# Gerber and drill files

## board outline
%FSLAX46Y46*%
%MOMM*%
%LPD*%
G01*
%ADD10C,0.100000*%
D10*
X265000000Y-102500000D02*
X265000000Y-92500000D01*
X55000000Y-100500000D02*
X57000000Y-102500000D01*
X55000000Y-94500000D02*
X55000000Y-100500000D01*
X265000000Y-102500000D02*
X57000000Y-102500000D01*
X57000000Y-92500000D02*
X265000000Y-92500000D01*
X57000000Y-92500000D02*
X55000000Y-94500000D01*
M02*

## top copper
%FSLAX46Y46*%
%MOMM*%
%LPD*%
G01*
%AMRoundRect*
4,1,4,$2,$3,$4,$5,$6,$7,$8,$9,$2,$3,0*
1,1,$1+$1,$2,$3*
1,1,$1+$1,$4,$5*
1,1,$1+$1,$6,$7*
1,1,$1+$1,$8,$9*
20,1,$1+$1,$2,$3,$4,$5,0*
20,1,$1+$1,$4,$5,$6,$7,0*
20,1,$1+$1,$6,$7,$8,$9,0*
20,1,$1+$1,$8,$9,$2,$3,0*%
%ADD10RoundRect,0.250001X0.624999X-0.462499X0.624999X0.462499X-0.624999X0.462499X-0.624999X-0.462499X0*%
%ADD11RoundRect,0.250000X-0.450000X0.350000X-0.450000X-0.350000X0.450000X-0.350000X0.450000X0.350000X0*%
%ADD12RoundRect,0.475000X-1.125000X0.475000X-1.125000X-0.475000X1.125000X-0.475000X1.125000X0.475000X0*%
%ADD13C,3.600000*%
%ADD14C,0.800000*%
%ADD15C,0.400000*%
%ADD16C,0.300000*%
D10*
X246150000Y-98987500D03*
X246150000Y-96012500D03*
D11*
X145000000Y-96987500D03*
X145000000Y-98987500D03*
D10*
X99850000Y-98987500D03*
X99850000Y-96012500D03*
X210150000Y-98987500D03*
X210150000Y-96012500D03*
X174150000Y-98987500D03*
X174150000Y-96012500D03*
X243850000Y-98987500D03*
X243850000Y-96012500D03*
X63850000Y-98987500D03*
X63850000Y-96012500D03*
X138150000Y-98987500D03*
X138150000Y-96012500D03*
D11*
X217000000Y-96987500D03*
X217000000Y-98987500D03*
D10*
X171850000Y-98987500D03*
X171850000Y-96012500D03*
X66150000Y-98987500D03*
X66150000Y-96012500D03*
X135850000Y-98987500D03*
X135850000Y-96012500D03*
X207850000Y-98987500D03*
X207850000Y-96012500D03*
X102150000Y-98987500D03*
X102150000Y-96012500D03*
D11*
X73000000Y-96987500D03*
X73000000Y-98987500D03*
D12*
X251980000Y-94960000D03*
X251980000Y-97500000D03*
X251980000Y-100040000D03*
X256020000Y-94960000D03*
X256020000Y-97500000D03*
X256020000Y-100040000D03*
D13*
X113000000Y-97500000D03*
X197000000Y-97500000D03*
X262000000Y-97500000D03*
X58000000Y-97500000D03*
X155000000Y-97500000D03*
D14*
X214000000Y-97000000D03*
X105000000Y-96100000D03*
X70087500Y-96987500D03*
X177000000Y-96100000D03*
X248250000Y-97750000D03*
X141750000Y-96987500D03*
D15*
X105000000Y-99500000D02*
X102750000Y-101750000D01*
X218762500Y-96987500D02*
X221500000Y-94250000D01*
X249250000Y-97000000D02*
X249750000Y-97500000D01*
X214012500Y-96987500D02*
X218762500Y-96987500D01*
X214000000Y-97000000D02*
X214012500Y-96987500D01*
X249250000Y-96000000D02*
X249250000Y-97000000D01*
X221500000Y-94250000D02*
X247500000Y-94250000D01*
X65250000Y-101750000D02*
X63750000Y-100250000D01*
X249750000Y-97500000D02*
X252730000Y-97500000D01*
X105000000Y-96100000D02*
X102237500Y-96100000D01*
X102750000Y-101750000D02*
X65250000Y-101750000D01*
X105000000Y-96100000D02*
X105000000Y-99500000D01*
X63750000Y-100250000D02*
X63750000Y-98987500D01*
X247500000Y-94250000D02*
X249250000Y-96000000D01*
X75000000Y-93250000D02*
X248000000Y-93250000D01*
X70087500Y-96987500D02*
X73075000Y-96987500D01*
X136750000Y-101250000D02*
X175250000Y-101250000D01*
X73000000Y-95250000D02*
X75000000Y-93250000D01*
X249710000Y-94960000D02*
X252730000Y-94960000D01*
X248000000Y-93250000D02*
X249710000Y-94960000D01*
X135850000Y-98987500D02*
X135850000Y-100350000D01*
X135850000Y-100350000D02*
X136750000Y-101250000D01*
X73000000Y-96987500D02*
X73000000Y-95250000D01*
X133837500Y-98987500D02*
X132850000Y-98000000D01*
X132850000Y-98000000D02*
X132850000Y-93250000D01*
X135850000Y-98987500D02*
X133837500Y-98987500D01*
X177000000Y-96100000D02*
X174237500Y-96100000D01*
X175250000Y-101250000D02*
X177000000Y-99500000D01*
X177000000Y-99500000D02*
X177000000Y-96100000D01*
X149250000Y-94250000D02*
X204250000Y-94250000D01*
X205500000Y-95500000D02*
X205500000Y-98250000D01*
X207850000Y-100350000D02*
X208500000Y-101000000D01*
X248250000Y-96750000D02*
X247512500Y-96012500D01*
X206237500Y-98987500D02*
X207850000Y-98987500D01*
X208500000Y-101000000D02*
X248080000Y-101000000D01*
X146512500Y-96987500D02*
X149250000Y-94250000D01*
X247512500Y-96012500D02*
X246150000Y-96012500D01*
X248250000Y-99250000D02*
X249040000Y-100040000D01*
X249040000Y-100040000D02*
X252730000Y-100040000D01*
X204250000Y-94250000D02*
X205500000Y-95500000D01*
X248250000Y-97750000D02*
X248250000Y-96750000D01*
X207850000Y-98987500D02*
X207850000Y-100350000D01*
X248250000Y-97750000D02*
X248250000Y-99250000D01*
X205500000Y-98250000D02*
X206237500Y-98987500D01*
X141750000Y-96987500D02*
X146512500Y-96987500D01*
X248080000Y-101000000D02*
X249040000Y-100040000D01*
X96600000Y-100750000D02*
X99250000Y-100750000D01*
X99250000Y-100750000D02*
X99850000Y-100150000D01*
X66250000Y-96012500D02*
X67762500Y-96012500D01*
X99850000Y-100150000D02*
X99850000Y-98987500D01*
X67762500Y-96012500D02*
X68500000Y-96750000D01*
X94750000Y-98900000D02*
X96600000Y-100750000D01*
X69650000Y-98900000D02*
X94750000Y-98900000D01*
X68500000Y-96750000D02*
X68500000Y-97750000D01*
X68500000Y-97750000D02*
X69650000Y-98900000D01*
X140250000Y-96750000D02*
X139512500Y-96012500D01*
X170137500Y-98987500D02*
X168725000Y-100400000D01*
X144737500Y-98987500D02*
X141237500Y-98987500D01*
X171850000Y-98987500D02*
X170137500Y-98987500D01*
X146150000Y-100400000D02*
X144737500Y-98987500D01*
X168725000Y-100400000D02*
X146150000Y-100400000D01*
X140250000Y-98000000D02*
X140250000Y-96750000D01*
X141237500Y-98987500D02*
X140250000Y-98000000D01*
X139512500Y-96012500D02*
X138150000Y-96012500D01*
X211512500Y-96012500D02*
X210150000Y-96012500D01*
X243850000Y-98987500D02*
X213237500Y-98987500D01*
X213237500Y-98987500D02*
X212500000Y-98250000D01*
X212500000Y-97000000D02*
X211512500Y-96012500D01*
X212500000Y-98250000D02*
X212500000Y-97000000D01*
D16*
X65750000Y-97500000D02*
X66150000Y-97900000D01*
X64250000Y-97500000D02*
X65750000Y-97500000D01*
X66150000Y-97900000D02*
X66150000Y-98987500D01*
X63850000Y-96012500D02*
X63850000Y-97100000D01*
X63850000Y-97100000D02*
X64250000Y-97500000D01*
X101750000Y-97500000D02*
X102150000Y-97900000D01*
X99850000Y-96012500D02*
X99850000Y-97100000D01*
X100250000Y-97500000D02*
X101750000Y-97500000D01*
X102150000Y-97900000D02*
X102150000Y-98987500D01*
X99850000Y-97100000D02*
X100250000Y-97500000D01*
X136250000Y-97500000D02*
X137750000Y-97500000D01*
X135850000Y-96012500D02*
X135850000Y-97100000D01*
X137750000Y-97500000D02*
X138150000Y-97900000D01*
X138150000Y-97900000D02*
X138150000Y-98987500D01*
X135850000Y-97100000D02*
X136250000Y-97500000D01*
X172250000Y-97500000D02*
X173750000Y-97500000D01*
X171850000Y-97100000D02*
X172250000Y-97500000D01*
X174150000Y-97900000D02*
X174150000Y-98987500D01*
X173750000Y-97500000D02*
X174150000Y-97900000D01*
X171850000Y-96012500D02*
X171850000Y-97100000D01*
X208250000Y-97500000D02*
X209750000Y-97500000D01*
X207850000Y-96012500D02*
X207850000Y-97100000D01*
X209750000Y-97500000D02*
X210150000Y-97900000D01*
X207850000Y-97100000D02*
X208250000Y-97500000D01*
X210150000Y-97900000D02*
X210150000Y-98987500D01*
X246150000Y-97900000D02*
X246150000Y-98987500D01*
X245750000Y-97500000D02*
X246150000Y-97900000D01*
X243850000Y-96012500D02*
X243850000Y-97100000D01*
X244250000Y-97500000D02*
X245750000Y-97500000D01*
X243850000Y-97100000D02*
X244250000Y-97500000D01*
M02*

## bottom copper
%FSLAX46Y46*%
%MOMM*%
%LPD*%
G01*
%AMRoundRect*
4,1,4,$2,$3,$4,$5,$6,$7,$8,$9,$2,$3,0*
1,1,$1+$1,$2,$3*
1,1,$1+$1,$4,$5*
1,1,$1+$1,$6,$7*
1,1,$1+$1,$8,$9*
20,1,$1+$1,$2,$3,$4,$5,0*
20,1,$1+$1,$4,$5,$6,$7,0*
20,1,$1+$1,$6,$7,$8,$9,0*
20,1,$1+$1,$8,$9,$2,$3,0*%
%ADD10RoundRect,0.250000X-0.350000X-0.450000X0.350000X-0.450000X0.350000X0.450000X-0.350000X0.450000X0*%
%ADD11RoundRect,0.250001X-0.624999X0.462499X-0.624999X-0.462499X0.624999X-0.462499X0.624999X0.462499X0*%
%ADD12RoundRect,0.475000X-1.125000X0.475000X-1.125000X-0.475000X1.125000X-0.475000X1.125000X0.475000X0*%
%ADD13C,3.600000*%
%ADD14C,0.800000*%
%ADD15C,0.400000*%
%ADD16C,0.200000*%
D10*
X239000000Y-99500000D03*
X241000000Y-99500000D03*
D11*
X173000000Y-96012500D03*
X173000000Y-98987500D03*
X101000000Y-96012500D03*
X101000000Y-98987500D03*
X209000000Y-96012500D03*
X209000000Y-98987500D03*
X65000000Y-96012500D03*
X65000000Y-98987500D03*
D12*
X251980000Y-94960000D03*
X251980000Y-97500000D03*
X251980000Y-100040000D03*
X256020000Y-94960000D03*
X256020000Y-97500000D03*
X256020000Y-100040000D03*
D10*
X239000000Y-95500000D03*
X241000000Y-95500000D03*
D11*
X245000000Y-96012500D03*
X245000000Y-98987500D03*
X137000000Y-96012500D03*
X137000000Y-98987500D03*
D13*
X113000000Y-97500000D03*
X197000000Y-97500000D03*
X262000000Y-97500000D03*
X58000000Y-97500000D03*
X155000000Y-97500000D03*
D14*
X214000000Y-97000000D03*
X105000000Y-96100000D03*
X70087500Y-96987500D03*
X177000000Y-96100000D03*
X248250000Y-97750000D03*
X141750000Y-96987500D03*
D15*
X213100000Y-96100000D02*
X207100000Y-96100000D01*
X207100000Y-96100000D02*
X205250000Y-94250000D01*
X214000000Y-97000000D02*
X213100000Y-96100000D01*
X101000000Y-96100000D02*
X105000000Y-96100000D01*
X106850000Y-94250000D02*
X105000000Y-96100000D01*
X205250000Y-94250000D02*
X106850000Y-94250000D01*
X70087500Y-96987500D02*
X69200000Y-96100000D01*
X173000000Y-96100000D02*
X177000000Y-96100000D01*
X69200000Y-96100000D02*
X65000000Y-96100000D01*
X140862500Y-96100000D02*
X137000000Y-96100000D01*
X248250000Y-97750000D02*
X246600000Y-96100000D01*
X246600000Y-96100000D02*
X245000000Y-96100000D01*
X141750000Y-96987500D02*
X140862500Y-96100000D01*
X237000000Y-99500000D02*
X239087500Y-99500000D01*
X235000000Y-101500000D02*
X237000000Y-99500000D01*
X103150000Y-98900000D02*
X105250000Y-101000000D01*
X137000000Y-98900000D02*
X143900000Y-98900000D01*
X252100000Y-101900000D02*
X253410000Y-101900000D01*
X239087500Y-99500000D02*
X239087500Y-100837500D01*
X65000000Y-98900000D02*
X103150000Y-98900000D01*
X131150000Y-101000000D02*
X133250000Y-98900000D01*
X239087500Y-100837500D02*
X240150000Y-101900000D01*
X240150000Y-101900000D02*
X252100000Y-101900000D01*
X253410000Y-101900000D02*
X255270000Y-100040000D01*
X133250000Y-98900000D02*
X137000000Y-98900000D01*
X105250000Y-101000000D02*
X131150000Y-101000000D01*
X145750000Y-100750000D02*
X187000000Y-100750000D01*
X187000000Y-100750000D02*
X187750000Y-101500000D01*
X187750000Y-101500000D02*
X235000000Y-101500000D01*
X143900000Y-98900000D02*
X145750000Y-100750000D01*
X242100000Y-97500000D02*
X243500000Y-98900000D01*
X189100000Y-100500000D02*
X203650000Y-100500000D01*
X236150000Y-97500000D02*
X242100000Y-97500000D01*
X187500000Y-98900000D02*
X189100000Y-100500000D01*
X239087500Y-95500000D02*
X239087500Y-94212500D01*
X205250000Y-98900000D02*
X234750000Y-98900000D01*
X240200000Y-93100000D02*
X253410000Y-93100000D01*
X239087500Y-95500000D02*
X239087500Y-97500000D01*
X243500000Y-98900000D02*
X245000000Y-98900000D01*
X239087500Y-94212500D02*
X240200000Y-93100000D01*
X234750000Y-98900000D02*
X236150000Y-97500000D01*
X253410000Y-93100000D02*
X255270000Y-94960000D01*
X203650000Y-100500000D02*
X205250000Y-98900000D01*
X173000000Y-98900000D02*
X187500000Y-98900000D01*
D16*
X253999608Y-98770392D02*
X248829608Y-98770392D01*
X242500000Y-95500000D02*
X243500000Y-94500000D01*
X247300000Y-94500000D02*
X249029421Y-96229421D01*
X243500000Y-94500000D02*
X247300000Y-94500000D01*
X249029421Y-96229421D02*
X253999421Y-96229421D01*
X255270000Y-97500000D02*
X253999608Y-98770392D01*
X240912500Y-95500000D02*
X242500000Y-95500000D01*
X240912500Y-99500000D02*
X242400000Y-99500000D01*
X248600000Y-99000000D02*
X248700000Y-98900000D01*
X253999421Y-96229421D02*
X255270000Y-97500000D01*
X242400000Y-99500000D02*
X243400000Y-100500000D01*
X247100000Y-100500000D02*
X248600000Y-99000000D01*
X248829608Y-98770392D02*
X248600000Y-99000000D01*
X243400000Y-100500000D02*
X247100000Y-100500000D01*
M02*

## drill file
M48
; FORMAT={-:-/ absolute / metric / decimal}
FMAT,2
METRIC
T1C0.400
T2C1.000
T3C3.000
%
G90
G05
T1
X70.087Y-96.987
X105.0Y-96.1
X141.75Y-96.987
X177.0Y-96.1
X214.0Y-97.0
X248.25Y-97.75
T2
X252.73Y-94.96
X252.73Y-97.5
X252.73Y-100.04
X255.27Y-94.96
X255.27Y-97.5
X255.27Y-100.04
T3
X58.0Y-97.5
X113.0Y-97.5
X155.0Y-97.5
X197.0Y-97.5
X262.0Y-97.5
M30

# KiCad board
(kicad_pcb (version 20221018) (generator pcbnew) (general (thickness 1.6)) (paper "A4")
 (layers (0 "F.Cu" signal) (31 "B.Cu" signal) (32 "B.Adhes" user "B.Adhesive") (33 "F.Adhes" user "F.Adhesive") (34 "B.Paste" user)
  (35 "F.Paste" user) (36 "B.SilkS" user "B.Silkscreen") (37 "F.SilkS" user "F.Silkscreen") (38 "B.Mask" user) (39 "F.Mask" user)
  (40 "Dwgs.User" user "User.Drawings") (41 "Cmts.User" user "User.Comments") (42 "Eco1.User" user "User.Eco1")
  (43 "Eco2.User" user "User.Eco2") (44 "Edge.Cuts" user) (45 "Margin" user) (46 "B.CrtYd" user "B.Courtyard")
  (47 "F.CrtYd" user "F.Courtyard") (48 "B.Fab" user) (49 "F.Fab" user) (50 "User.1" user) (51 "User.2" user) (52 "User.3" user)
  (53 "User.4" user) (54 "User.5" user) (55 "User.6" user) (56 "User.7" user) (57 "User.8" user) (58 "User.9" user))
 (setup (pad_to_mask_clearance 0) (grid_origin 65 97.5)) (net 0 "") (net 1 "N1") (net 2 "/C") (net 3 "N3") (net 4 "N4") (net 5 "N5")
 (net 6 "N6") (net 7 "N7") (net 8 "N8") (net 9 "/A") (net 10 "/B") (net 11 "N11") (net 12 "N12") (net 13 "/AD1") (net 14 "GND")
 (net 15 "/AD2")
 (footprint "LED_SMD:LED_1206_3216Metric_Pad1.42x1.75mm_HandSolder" (layer "F.Cu") (at 246.15 97.5 90)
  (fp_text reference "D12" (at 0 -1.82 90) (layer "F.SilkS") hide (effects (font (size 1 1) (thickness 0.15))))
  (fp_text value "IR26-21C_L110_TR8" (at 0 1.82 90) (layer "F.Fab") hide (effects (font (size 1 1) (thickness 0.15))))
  (pad "1" smd roundrect (at -1.4875 0 90) (size 1.425 1.75) (layers "F.Cu" "F.Paste" "F.Mask") (roundrect_rratio 0.175439) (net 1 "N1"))
  (pad "2" smd roundrect (at 1.4875 0 90) (size 1.425 1.75) (layers "F.Cu" "F.Paste" "F.Mask") (roundrect_rratio 0.175439) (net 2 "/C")))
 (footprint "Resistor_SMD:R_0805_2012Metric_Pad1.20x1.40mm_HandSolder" (layer "F.Cu") (at 145 97.9875 -90)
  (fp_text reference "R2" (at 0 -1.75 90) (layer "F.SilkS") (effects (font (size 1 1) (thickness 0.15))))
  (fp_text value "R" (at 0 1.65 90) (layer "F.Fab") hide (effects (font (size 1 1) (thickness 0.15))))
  (pad "1" smd roundrect (at -1 0 270) (size 1.2 1.4) (layers "F.Cu" "F.Paste" "F.Mask") (roundrect_rratio 0.208333) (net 2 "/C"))
  (pad "2" smd roundrect (at 1 0 270) (size 1.2 1.4) (layers "F.Cu" "F.Paste" "F.Mask") (roundrect_rratio 0.208333) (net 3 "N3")))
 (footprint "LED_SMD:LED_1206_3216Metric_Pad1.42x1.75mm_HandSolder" (layer "F.Cu") (at 99.85 97.5 90)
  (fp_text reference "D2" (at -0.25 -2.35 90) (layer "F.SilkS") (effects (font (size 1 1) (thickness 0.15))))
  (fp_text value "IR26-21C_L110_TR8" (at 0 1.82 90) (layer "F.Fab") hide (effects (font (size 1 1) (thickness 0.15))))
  (pad "1" smd roundrect (at -1.4875 0 90) (size 1.425 1.75) (layers "F.Cu" "F.Paste" "F.Mask") (roundrect_rratio 0.175439) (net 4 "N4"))
  (pad "2" smd roundrect (at 1.4875 0 90) (size 1.425 1.75) (layers "F.Cu" "F.Paste" "F.Mask") (roundrect_rratio 0.175439) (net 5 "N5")))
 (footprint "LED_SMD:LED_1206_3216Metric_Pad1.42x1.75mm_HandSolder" (layer "F.Cu") (at 210.15 97.5 90)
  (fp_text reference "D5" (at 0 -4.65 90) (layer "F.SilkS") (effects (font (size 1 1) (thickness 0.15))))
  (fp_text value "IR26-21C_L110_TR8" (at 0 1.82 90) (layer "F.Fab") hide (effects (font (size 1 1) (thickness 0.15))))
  (pad "1" smd roundrect (at -1.4875 0 90) (size 1.425 1.75) (layers "F.Cu" "F.Paste" "F.Mask") (roundrect_rratio 0.175439) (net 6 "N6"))
  (pad "2" smd roundrect (at 1.4875 0 90) (size 1.425 1.75) (layers "F.Cu" "F.Paste" "F.Mask") (roundrect_rratio 0.175439) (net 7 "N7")))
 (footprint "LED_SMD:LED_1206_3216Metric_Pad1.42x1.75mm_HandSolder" (layer "F.Cu") (at 174.15 97.5 90)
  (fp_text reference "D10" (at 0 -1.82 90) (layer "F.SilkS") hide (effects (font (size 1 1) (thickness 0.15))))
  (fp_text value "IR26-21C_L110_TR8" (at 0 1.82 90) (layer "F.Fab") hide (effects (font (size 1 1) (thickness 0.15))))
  (pad "1" smd roundrect (at -1.4875 0 90) (size 1.425 1.75) (layers "F.Cu" "F.Paste" "F.Mask") (roundrect_rratio 0.175439) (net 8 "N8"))
  (pad "2" smd roundrect (at 1.4875 0 90) (size 1.425 1.75) (layers "F.Cu" "F.Paste" "F.Mask") (roundrect_rratio 0.175439) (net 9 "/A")))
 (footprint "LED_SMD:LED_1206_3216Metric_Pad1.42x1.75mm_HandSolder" (layer "F.Cu") (at 243.85 97.5 90)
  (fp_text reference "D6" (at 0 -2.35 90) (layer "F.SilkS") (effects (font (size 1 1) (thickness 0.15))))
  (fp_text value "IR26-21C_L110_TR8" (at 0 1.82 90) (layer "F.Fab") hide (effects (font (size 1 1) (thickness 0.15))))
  (pad "1" smd roundrect (at -1.4875 0 90) (size 1.425 1.75) (layers "F.Cu" "F.Paste" "F.Mask") (roundrect_rratio 0.175439) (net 7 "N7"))
  (pad "2" smd roundrect (at 1.4875 0 90) (size 1.425 1.75) (layers "F.Cu" "F.Paste" "F.Mask") (roundrect_rratio 0.175439) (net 1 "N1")))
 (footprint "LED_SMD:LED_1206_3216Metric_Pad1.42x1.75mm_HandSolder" (layer "F.Cu") (at 63.85 97.5 90)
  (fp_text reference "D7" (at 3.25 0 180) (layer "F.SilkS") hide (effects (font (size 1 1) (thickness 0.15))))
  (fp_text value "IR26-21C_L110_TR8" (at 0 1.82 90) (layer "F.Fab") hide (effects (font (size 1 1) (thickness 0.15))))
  (pad "1" smd roundrect (at -1.4875 0 90) (size 1.425 1.75) (layers "F.Cu" "F.Paste" "F.Mask") (roundrect_rratio 0.175439) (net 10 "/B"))
  (pad "2" smd roundrect (at 1.4875 0 90) (size 1.425 1.75) (layers "F.Cu" "F.Paste" "F.Mask") (roundrect_rratio 0.175439) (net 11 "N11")))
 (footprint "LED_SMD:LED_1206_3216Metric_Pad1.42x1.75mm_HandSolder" (layer "F.Cu") (at 138.15 97.5 90)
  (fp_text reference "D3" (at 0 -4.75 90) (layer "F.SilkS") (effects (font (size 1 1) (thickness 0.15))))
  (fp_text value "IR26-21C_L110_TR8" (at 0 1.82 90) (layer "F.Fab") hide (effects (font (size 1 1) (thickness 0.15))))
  (pad "1" smd roundrect (at -1.4875 0 90) (size 1.425 1.75) (layers "F.Cu" "F.Paste" "F.Mask") (roundrect_rratio 0.175439) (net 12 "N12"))
  (pad "2" smd roundrect (at 1.4875 0 90) (size 1.425 1.75) (layers "F.Cu" "F.Paste" "F.Mask") (roundrect_rratio 0.175439) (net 3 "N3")))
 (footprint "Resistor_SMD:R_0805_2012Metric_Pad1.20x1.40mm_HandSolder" (layer "F.Cu") (at 217 97.9875 -90)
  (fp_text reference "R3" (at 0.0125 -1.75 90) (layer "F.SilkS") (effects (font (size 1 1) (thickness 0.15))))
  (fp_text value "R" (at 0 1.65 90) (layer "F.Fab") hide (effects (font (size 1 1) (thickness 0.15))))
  (pad "1" smd roundrect (at -1 0 270) (size 1.2 1.4) (layers "F.Cu" "F.Paste" "F.Mask") (roundrect_rratio 0.208333) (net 10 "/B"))
  (pad "2" smd roundrect (at 1 0 270) (size 1.2 1.4) (layers "F.Cu" "F.Paste" "F.Mask") (roundrect_rratio 0.208333) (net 7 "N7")))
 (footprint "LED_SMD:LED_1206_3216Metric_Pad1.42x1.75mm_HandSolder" (layer "F.Cu") (at 171.85 97.5 90)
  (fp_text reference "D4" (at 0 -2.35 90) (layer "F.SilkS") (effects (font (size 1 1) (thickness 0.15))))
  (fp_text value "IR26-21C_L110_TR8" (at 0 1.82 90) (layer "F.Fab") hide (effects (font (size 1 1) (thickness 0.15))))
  (pad "1" smd roundrect (at -1.4875 0 90) (size 1.425 1.75) (layers "F.Cu" "F.Paste" "F.Mask") (roundrect_rratio 0.175439) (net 3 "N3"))
  (pad "2" smd roundrect (at 1.4875 0 90) (size 1.425 1.75) (layers "F.Cu" "F.Paste" "F.Mask") (roundrect_rratio 0.175439) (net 8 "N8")))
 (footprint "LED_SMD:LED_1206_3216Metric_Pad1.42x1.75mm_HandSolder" (layer "F.Cu") (at 66.15 97.5 90)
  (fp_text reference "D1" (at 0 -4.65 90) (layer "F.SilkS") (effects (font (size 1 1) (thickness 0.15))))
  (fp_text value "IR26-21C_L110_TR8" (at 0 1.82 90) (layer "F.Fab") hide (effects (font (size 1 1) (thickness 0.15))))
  (pad "1" smd roundrect (at -1.4875 0 90) (size 1.425 1.75) (layers "F.Cu" "F.Paste" "F.Mask") (roundrect_rratio 0.175439) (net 11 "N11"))
  (pad "2" smd roundrect (at 1.4875 0 90) (size 1.425 1.75) (layers "F.Cu" "F.Paste" "F.Mask") (roundrect_rratio 0.175439) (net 4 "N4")))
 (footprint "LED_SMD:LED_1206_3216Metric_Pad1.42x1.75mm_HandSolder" (layer "F.Cu") (at 135.85 97.5 90)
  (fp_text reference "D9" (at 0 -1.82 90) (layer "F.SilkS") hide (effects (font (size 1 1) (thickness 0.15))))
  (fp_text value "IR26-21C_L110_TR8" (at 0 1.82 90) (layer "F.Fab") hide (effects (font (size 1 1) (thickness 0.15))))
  (pad "1" smd roundrect (at -1.4875 0 90) (size 1.425 1.75) (layers "F.Cu" "F.Paste" "F.Mask") (roundrect_rratio 0.175439) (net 9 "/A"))
  (pad "2" smd roundrect (at 1.4875 0 90) (size 1.425 1.75) (layers "F.Cu" "F.Paste" "F.Mask") (roundrect_rratio 0.175439) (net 12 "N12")))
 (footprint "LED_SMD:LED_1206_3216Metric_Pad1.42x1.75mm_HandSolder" (layer "F.Cu") (at 207.85 97.5 90)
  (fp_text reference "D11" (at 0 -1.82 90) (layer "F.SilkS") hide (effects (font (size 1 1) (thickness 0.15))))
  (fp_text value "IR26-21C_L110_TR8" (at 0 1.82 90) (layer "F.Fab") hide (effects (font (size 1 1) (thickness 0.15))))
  (pad "1" smd roundrect (at -1.4875 0 90) (size 1.425 1.75) (layers "F.Cu" "F.Paste" "F.Mask") (roundrect_rratio 0.175439) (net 2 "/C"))
  (pad "2" smd roundrect (at 1.4875 0 90) (size 1.425 1.75) (layers "F.Cu" "F.Paste" "F.Mask") (roundrect_rratio 0.175439) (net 6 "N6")))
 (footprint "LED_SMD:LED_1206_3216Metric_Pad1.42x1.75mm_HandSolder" (layer "F.Cu") (at 102.15 97.5 90)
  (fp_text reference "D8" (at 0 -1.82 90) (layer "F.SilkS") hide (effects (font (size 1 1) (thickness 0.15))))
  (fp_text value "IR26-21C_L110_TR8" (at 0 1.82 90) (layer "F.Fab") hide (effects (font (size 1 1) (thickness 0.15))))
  (pad "1" smd roundrect (at -1.4875 0 90) (size 1.425 1.75) (layers "F.Cu" "F.Paste" "F.Mask") (roundrect_rratio 0.175439) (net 5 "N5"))
  (pad "2" smd roundrect (at 1.4875 0 90) (size 1.425 1.75) (layers "F.Cu" "F.Paste" "F.Mask") (roundrect_rratio 0.175439) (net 10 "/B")))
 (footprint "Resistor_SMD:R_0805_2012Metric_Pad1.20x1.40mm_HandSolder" (layer "F.Cu") (at 73 97.9875 -90)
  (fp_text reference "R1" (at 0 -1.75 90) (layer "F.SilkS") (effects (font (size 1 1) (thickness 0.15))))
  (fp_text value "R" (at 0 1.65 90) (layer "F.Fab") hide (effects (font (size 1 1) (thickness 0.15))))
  (pad "1" smd roundrect (at -1 0 270) (size 1.2 1.4) (layers "F.Cu" "F.Paste" "F.Mask") (roundrect_rratio 0.208333) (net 9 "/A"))
  (pad "2" smd roundrect (at 1 0 270) (size 1.2 1.4) (layers "F.Cu" "F.Paste" "F.Mask") (roundrect_rratio 0.208333) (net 4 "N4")))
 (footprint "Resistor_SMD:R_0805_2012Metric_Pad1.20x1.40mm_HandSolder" (layer "B.Cu") (at 240 99.5)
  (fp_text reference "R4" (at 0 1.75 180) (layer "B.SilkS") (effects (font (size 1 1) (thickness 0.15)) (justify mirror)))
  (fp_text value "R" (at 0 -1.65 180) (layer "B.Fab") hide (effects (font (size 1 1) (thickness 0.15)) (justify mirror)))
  (pad "1" smd roundrect (at -1 0) (size 1.2 1.4) (layers "B.Cu" "B.Paste" "B.Mask") (roundrect_rratio 0.208333) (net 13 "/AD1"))
  (pad "2" smd roundrect (at 1 0) (size 1.2 1.4) (layers "B.Cu" "B.Paste" "B.Mask") (roundrect_rratio 0.208333) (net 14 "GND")))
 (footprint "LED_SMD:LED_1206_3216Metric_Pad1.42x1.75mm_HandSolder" (layer "B.Cu") (at 173 97.5 -90)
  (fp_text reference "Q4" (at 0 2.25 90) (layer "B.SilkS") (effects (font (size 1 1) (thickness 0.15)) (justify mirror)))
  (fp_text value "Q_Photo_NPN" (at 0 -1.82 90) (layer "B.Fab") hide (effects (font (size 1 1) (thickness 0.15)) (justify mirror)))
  (pad "1" smd roundrect (at -1.4875 0 270) (size 1.425 1.75) (layers "B.Cu" "B.Paste" "B.Mask") (roundrect_rratio 0.175439) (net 9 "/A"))
  (pad "2" smd roundrect (at 1.4875 0 270) (size 1.425 1.75) (layers "B.Cu" "B.Paste" "B.Mask") (roundrect_rratio 0.175439) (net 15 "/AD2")))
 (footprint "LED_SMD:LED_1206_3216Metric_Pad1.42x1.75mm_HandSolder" (layer "B.Cu") (at 101 97.5 -90)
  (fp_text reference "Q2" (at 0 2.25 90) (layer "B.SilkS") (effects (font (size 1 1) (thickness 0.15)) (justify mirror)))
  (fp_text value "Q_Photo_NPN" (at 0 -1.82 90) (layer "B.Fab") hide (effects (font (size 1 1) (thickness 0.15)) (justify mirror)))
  (pad "1" smd roundrect (at -1.4875 0 270) (size 1.425 1.75) (layers "B.Cu" "B.Paste" "B.Mask") (roundrect_rratio 0.175439) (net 10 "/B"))
  (pad "2" smd roundrect (at 1.4875 0 270) (size 1.425 1.75) (layers "B.Cu" "B.Paste" "B.Mask") (roundrect_rratio 0.175439) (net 13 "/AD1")))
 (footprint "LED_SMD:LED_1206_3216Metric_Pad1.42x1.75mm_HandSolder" (layer "B.Cu") (at 209 97.5 -90)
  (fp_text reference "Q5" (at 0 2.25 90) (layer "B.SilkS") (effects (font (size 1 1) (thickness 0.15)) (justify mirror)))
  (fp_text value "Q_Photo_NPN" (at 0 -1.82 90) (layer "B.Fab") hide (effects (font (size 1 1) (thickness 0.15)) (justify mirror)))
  (pad "1" smd roundrect (at -1.4875 0 270) (size 1.425 1.75) (layers "B.Cu" "B.Paste" "B.Mask") (roundrect_rratio 0.175439) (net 10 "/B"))
  (pad "2" smd roundrect (at 1.4875 0 270) (size 1.425 1.75) (layers "B.Cu" "B.Paste" "B.Mask") (roundrect_rratio 0.175439) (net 15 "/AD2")))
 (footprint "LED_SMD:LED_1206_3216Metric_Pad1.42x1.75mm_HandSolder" (layer "B.Cu") (at 65 97.5 -90)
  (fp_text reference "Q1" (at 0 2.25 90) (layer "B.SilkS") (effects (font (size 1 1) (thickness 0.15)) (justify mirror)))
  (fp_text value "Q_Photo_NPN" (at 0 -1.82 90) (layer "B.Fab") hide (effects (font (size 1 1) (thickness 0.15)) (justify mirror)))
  (pad "1" smd roundrect (at -1.4875 0 270) (size 1.425 1.75) (layers "B.Cu" "B.Paste" "B.Mask") (roundrect_rratio 0.175439) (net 9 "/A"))
  (pad "2" smd roundrect (at 1.4875 0 270) (size 1.425 1.75) (layers "B.Cu" "B.Paste" "B.Mask") (roundrect_rratio 0.175439) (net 13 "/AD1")))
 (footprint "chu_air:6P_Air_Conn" (layer "B.Cu") (at 254 97.5 -90)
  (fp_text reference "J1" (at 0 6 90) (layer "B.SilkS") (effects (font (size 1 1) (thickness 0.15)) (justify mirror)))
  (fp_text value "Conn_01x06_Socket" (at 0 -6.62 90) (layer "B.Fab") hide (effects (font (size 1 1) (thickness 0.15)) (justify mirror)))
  (pad "1" thru_hole roundrect (at -2.54 1.27 270) (size 1.9 3.2) (drill 1 (offset 0 0.75)) (layers "*.Cu" "*.Mask") (roundrect_rratio 0.25)
   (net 9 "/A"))
  (pad "2" thru_hole roundrect (at 0 1.27 270) (size 1.9 3.2) (drill 1 (offset 0 0.75)) (layers "*.Cu" "*.Mask") (roundrect_rratio 0.25)
   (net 10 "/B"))
  (pad "3" thru_hole roundrect (at 2.54 1.27 270) (size 1.9 3.2) (drill 1 (offset 0 0.75)) (layers "*.Cu" "*.Mask") (roundrect_rratio 0.25)
   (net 2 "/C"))
  (pad "4" thru_hole roundrect (at -2.54 -1.27 270) (size 1.9 3.2) (drill 1 (offset 0 -0.75)) (layers "*.Cu" "*.Mask")
   (roundrect_rratio 0.25) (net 15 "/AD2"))
  (pad "5" thru_hole roundrect (at 0 -1.27 270) (size 1.9 3.2) (drill 1 (offset 0 -0.75)) (layers "*.Cu" "*.Mask") (roundrect_rratio 0.25)
   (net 14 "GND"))
  (pad "6" thru_hole roundrect (at 2.54 -1.27 270) (size 1.9 3.2) (drill 1 (offset 0 -0.75)) (layers "*.Cu" "*.Mask")
   (roundrect_rratio 0.25) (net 13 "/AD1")))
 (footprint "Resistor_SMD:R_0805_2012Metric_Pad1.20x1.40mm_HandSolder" (layer "B.Cu") (at 240 95.5)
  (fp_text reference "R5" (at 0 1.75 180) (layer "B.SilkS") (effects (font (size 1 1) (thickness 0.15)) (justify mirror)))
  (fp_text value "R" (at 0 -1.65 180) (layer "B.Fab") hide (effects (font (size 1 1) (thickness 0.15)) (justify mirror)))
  (pad "1" smd roundrect (at -1 0) (size 1.2 1.4) (layers "B.Cu" "B.Paste" "B.Mask") (roundrect_rratio 0.208333) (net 15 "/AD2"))
  (pad "2" smd roundrect (at 1 0) (size 1.2 1.4) (layers "B.Cu" "B.Paste" "B.Mask") (roundrect_rratio 0.208333) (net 14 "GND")))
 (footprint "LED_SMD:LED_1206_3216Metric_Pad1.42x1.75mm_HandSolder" (layer "B.Cu") (at 245 97.5 -90)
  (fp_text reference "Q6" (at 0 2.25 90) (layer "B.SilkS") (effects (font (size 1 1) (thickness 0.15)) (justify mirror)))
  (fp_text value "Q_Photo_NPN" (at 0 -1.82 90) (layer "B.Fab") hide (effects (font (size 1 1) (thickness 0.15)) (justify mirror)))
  (pad "1" smd roundrect (at -1.4875 0 270) (size 1.425 1.75) (layers "B.Cu" "B.Paste" "B.Mask") (roundrect_rratio 0.175439) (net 2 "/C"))
  (pad "2" smd roundrect (at 1.4875 0 270) (size 1.425 1.75) (layers "B.Cu" "B.Paste" "B.Mask") (roundrect_rratio 0.175439) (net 15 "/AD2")))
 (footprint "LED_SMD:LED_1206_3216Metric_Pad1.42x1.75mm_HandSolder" (layer "B.Cu") (at 137 97.5 -90)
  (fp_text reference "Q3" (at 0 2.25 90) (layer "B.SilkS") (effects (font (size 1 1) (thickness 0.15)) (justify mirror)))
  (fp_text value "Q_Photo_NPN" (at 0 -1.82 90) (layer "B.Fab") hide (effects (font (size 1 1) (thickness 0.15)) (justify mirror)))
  (pad "1" smd roundrect (at -1.4875 0 270) (size 1.425 1.75) (layers "B.Cu" "B.Paste" "B.Mask") (roundrect_rratio 0.175439) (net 2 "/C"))
  (pad "2" smd roundrect (at 1.4875 0 270) (size 1.425 1.75) (layers "B.Cu" "B.Paste" "B.Mask") (roundrect_rratio 0.175439) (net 13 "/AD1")))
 (gr_line (start 265 102.5) (end 265 92.5) (stroke (width 0.1) (type default)) (layer "Edge.Cuts"))
 (gr_line (start 55 100.5) (end 57 102.5) (stroke (width 0.1) (type default)) (layer "Edge.Cuts"))
 (gr_line (start 55 94.5) (end 55 100.5) (stroke (width 0.1) (type default)) (layer "Edge.Cuts"))
 (gr_line (start 265 102.5) (end 57 102.5) (stroke (width 0.1) (type default)) (layer "Edge.Cuts"))
 (gr_line (start 57 92.5) (end 265 92.5) (stroke (width 0.1) (type default)) (layer "Edge.Cuts"))
 (gr_line (start 57 92.5) (end 55 94.5) (stroke (width 0.1) (type default)) (layer "Edge.Cuts"))
 (via (at 113 97.5) (size 3.6) (drill 3) (layers "F.Cu" "B.Cu") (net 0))
 (via (at 197 97.5) (size 3.6) (drill 3) (layers "F.Cu" "B.Cu") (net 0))
 (via (at 262 97.5) (size 3.6) (drill 3) (layers "F.Cu" "B.Cu") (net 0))
 (via (at 58 97.5) (size 3.6) (drill 3) (layers "F.Cu" "B.Cu") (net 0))
 (via (at 155 97.5) (size 3.6) (drill 3) (layers "F.Cu" "B.Cu") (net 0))
 (segment (start 105 99.5) (end 102.75 101.75) (width 0.4) (layer "F.Cu") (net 10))
 (segment (start 218.7625 96.9875) (end 221.5 94.25) (width 0.4) (layer "F.Cu") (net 10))
 (segment (start 249.25 97) (end 249.75 97.5) (width 0.4) (layer "F.Cu") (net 10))
 (segment (start 214.0125 96.9875) (end 218.7625 96.9875) (width 0.4) (layer "F.Cu") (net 10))
 (segment (start 214 97) (end 214.0125 96.9875) (width 0.4) (layer "F.Cu") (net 10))
 (segment (start 249.25 96) (end 249.25 97) (width 0.4) (layer "F.Cu") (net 10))
 (segment (start 221.5 94.25) (end 247.5 94.25) (width 0.4) (layer "F.Cu") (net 10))
 (segment (start 65.25 101.75) (end 63.75 100.25) (width 0.4) (layer "F.Cu") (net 10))
 (segment (start 249.75 97.5) (end 252.73 97.5) (width 0.4) (layer "F.Cu") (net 10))
 (segment (start 105 96.1) (end 102.2375 96.1) (width 0.4) (layer "F.Cu") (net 10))
 (segment (start 102.75 101.75) (end 65.25 101.75) (width 0.4) (layer "F.Cu") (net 10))
 (segment (start 105 96.1) (end 105 99.5) (width 0.4) (layer "F.Cu") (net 10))
 (segment (start 63.75 100.25) (end 63.75 98.9875) (width 0.4) (layer "F.Cu") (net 10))
 (segment (start 247.5 94.25) (end 249.25 96) (width 0.4) (layer "F.Cu") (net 10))
 (via (at 214 97) (size 0.8) (drill 0.4) (layers "F.Cu" "B.Cu") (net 10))
 (via (at 105 96.1) (size 0.8) (drill 0.4) (layers "F.Cu" "B.Cu") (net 10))
 (segment (start 213.1 96.1) (end 207.1 96.1) (width 0.4) (layer "B.Cu") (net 10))
 (segment (start 207.1 96.1) (end 205.25 94.25) (width 0.4) (layer "B.Cu") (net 10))
 (segment (start 214 97) (end 213.1 96.1) (width 0.4) (layer "B.Cu") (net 10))
 (segment (start 101 96.1) (end 105 96.1) (width 0.4) (layer "B.Cu") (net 10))
 (segment (start 106.85 94.25) (end 105 96.1) (width 0.4) (layer "B.Cu") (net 10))
 (segment (start 205.25 94.25) (end 106.85 94.25) (width 0.4) (layer "B.Cu") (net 10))
 (segment (start 75 93.25) (end 248 93.25) (width 0.4) (layer "F.Cu") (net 9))
 (segment (start 70.0875 96.9875) (end 73.075 96.9875) (width 0.4) (layer "F.Cu") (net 9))
 (segment (start 136.75 101.25) (end 175.25 101.25) (width 0.4) (layer "F.Cu") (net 9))
 (segment (start 73 95.25) (end 75 93.25) (width 0.4) (layer "F.Cu") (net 9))
 (segment (start 249.71 94.96) (end 252.73 94.96) (width 0.4) (layer "F.Cu") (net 9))
 (segment (start 248 93.25) (end 249.71 94.96) (width 0.4) (layer "F.Cu") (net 9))
 (segment (start 135.85 98.9875) (end 135.85 100.35) (width 0.4) (layer "F.Cu") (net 9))
 (segment (start 135.85 100.35) (end 136.75 101.25) (width 0.4) (layer "F.Cu") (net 9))
 (segment (start 73 96.9875) (end 73 95.25) (width 0.4) (layer "F.Cu") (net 9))
 (segment (start 133.8375 98.9875) (end 132.85 98) (width 0.4) (layer "F.Cu") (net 9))
 (segment (start 132.85 98) (end 132.85 93.25) (width 0.4) (layer "F.Cu") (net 9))
 (segment (start 135.85 98.9875) (end 133.8375 98.9875) (width 0.4) (layer "F.Cu") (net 9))
 (segment (start 177 96.1) (end 174.2375 96.1) (width 0.4) (layer "F.Cu") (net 9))
 (segment (start 175.25 101.25) (end 177 99.5) (width 0.4) (layer "F.Cu") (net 9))
 (segment (start 177 99.5) (end 177 96.1) (width 0.4) (layer "F.Cu") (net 9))
 (via (at 70.0875 96.9875) (size 0.8) (drill 0.4) (layers "F.Cu" "B.Cu") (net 9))
 (via (at 177 96.1) (size 0.8) (drill 0.4) (layers "F.Cu" "B.Cu") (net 9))
 (segment (start 70.0875 96.9875) (end 69.2 96.1) (width 0.4) (layer "B.Cu") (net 9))
 (segment (start 173 96.1) (end 177 96.1) (width 0.4) (layer "B.Cu") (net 9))
 (segment (start 69.2 96.1) (end 65 96.1) (width 0.4) (layer "B.Cu") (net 9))
 (segment (start 149.25 94.25) (end 204.25 94.25) (width 0.4) (layer "F.Cu") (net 2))
 (segment (start 205.5 95.5) (end 205.5 98.25) (width 0.4) (layer "F.Cu") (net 2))
 (segment (start 207.85 100.35) (end 208.5 101) (width 0.4) (layer "F.Cu") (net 2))
 (segment (start 248.25 96.75) (end 247.5125 96.0125) (width 0.4) (layer "F.Cu") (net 2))
 (segment (start 206.2375 98.9875) (end 207.85 98.9875) (width 0.4) (layer "F.Cu") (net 2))
 (segment (start 208.5 101) (end 248.08 101) (width 0.4) (layer "F.Cu") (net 2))
 (segment (start 146.5125 96.9875) (end 149.25 94.25) (width 0.4) (layer "F.Cu") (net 2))
 (segment (start 247.5125 96.0125) (end 246.15 96.0125) (width 0.4) (layer "F.Cu") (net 2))
 (segment (start 248.25 99.25) (end 249.04 100.04) (width 0.4) (layer "F.Cu") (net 2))
 (segment (start 249.04 100.04) (end 252.73 100.04) (width 0.4) (layer "F.Cu") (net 2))
 (segment (start 204.25 94.25) (end 205.5 95.5) (width 0.4) (layer "F.Cu") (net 2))
 (segment (start 248.25 97.75) (end 248.25 96.75) (width 0.4) (layer "F.Cu") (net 2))
 (segment (start 207.85 98.9875) (end 207.85 100.35) (width 0.4) (layer "F.Cu") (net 2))
 (segment (start 248.25 97.75) (end 248.25 99.25) (width 0.4) (layer "F.Cu") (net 2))
 (segment (start 205.5 98.25) (end 206.2375 98.9875) (width 0.4) (layer "F.Cu") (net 2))
 (segment (start 141.75 96.9875) (end 146.5125 96.9875) (width 0.4) (layer "F.Cu") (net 2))
 (segment (start 248.08 101) (end 249.04 100.04) (width 0.4) (layer "F.Cu") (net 2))
 (via (at 248.25 97.75) (size 0.8) (drill 0.4) (layers "F.Cu" "B.Cu") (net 2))
 (via (at 141.75 96.9875) (size 0.8) (drill 0.4) (layers "F.Cu" "B.Cu") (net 2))
 (segment (start 140.8625 96.1) (end 137 96.1) (width 0.4) (layer "B.Cu") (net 2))
 (segment (start 248.25 97.75) (end 246.6 96.1) (width 0.4) (layer "B.Cu") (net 2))
 (segment (start 246.6 96.1) (end 245 96.1) (width 0.4) (layer "B.Cu") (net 2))
 (segment (start 141.75 96.9875) (end 140.8625 96.1) (width 0.4) (layer "B.Cu") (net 2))
 (segment (start 237 99.5) (end 239.0875 99.5) (width 0.4) (layer "B.Cu") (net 13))
 (segment (start 235 101.5) (end 237 99.5) (width 0.4) (layer "B.Cu") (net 13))
 (segment (start 103.15 98.9) (end 105.25 101) (width 0.4) (layer "B.Cu") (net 13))
 (segment (start 137 98.9) (end 143.9 98.9) (width 0.4) (layer "B.Cu") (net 13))
 (segment (start 252.1 101.9) (end 253.41 101.9) (width 0.4) (layer "B.Cu") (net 13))
 (segment (start 239.0875 99.5) (end 239.0875 100.8375) (width 0.4) (layer "B.Cu") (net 13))
 (segment (start 65 98.9) (end 103.15 98.9) (width 0.4) (layer "B.Cu") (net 13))
 (segment (start 131.15 101) (end 133.25 98.9) (width 0.4) (layer "B.Cu") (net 13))
 (segment (start 239.0875 100.8375) (end 240.15 101.9) (width 0.4) (layer "B.Cu") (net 13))
 (segment (start 240.15 101.9) (end 252.1 101.9) (width 0.4) (layer "B.Cu") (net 13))
 (segment (start 253.41 101.9) (end 255.27 100.04) (width 0.4) (layer "B.Cu") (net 13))
 (segment (start 133.25 98.9) (end 137 98.9) (width 0.4) (layer "B.Cu") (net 13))
 (segment (start 105.25 101) (end 131.15 101) (width 0.4) (layer "B.Cu") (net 13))
 (segment (start 145.75 100.75) (end 187 100.75) (width 0.4) (layer "B.Cu") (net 13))
 (segment (start 187 100.75) (end 187.75 101.5) (width 0.4) (layer "B.Cu") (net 13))
 (segment (start 187.75 101.5) (end 235 101.5) (width 0.4) (layer "B.Cu") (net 13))
 (segment (start 143.9 98.9) (end 145.75 100.75) (width 0.4) (layer "B.Cu") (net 13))
 (segment (start 242.1 97.5) (end 243.5 98.9) (width 0.4) (layer "B.Cu") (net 15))
 (segment (start 189.1 100.5) (end 203.65 100.5) (width 0.4) (layer "B.Cu") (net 15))
 (segment (start 236.15 97.5) (end 242.1 97.5) (width 0.4) (layer "B.Cu") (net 15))
 (segment (start 187.5 98.9) (end 189.1 100.5) (width 0.4) (layer "B.Cu") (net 15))
 (segment (start 239.0875 95.5) (end 239.0875 94.2125) (width 0.4) (layer "B.Cu") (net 15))
 (segment (start 205.25 98.9) (end 234.75 98.9) (width 0.4) (layer "B.Cu") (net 15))
 (segment (start 240.2 93.1) (end 253.41 93.1) (width 0.4) (layer "B.Cu") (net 15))
 (segment (start 239.0875 95.5) (end 239.0875 97.5) (width 0.4) (layer "B.Cu") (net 15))
 (segment (start 243.5 98.9) (end 245 98.9) (width 0.4) (layer "B.Cu") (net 15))
 (segment (start 239.0875 94.2125) (end 240.2 93.1) (width 0.4) (layer "B.Cu") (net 15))
 (segment (start 234.75 98.9) (end 236.15 97.5) (width 0.4) (layer "B.Cu") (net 15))
 (segment (start 253.41 93.1) (end 255.27 94.96) (width 0.4) (layer "B.Cu") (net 15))
 (segment (start 203.65 100.5) (end 205.25 98.9) (width 0.4) (layer "B.Cu") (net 15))
 (segment (start 173 98.9) (end 187.5 98.9) (width 0.4) (layer "B.Cu") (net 15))
 (segment (start 253.999608 98.770392) (end 248.829608 98.770392) (width 0.2) (layer "B.Cu") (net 14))
 (segment (start 242.5 95.5) (end 243.5 94.5) (width 0.2) (layer "B.Cu") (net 14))
 (segment (start 247.3 94.5) (end 249.029421 96.229421) (width 0.2) (layer "B.Cu") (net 14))
 (segment (start 243.5 94.5) (end 247.3 94.5) (width 0.2) (layer "B.Cu") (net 14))
 (segment (start 249.029421 96.229421) (end 253.999421 96.229421) (width 0.2) (layer "B.Cu") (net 14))
 (segment (start 255.27 97.5) (end 253.999608 98.770392) (width 0.2) (layer "B.Cu") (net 14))
 (segment (start 240.9125 95.5) (end 242.5 95.5) (width 0.2) (layer "B.Cu") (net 14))
 (segment (start 240.9125 99.5) (end 242.4 99.5) (width 0.2) (layer "B.Cu") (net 14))
 (segment (start 248.6 99) (end 248.7 98.9) (width 0.2) (layer "B.Cu") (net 14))
 (segment (start 253.999421 96.229421) (end 255.27 97.5) (width 0.2) (layer "B.Cu") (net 14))
 (segment (start 242.4 99.5) (end 243.4 100.5) (width 0.2) (layer "B.Cu") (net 14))
 (segment (start 247.1 100.5) (end 248.6 99) (width 0.2) (layer "B.Cu") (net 14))
 (segment (start 248.829608 98.770392) (end 248.6 99) (width 0.2) (layer "B.Cu") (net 14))
 (segment (start 243.4 100.5) (end 247.1 100.5) (width 0.2) (layer "B.Cu") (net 14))
 (segment (start 96.6 100.75) (end 99.25 100.75) (width 0.4) (layer "F.Cu") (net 4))
 (segment (start 99.25 100.75) (end 99.85 100.15) (width 0.4) (layer "F.Cu") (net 4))
 (segment (start 66.25 96.0125) (end 67.7625 96.0125) (width 0.4) (layer "F.Cu") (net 4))
 (segment (start 99.85 100.15) (end 99.85 98.9875) (width 0.4) (layer "F.Cu") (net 4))
 (segment (start 67.7625 96.0125) (end 68.5 96.75) (width 0.4) (layer "F.Cu") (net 4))
 (segment (start 94.75 98.9) (end 96.6 100.75) (width 0.4) (layer "F.Cu") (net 4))
 (segment (start 69.65 98.9) (end 94.75 98.9) (width 0.4) (layer "F.Cu") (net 4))
 (segment (start 68.5 96.75) (end 68.5 97.75) (width 0.4) (layer "F.Cu") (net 4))
 (segment (start 68.5 97.75) (end 69.65 98.9) (width 0.4) (layer "F.Cu") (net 4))
 (segment (start 140.25 96.75) (end 139.5125 96.0125) (width 0.4) (layer "F.Cu") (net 3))
 (segment (start 170.1375 98.9875) (end 168.725 100.4) (width 0.4) (layer "F.Cu") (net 3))
 (segment (start 144.7375 98.9875) (end 141.2375 98.9875) (width 0.4) (layer "F.Cu") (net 3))
 (segment (start 171.85 98.9875) (end 170.1375 98.9875) (width 0.4) (layer "F.Cu") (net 3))
 (segment (start 146.15 100.4) (end 144.7375 98.9875) (width 0.4) (layer "F.Cu") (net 3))
 (segment (start 168.725 100.4) (end 146.15 100.4) (width 0.4) (layer "F.Cu") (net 3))
 (segment (start 140.25 98) (end 140.25 96.75) (width 0.4) (layer "F.Cu") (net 3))
 (segment (start 141.2375 98.9875) (end 140.25 98) (width 0.4) (layer "F.Cu") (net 3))
 (segment (start 139.5125 96.0125) (end 138.15 96.0125) (width 0.4) (layer "F.Cu") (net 3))
 (segment (start 211.5125 96.0125) (end 210.15 96.0125) (width 0.4) (layer "F.Cu") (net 7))
 (segment (start 243.85 98.9875) (end 213.2375 98.9875) (width 0.4) (layer "F.Cu") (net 7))
 (segment (start 213.2375 98.9875) (end 212.5 98.25) (width 0.4) (layer "F.Cu") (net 7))
 (segment (start 212.5 97) (end 211.5125 96.0125) (width 0.4) (layer "F.Cu") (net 7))
 (segment (start 212.5 98.25) (end 212.5 97) (width 0.4) (layer "F.Cu") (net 7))
 (segment (start 65.75 97.5) (end 66.15 97.9) (width 0.3) (layer "F.Cu") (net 11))
 (segment (start 64.25 97.5) (end 65.75 97.5) (width 0.3) (layer "F.Cu") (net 11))
 (segment (start 66.15 97.9) (end 66.15 98.9875) (width 0.3) (layer "F.Cu") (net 11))
 (segment (start 63.85 96.0125) (end 63.85 97.1) (width 0.3) (layer "F.Cu") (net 11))
 (segment (start 63.85 97.1) (end 64.25 97.5) (width 0.3) (layer "F.Cu") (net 11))
 (segment (start 101.75 97.5) (end 102.15 97.9) (width 0.3) (layer "F.Cu") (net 5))
 (segment (start 99.85 96.0125) (end 99.85 97.1) (width 0.3) (layer "F.Cu") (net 5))
 (segment (start 100.25 97.5) (end 101.75 97.5) (width 0.3) (layer "F.Cu") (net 5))
 (segment (start 102.15 97.9) (end 102.15 98.9875) (width 0.3) (layer "F.Cu") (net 5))
 (segment (start 99.85 97.1) (end 100.25 97.5) (width 0.3) (layer "F.Cu") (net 5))
 (segment (start 136.25 97.5) (end 137.75 97.5) (width 0.3) (layer "F.Cu") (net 12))
 (segment (start 135.85 96.0125) (end 135.85 97.1) (width 0.3) (layer "F.Cu") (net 12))
 (segment (start 137.75 97.5) (end 138.15 97.9) (width 0.3) (layer "F.Cu") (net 12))
 (segment (start 138.15 97.9) (end 138.15 98.9875) (width 0.3) (layer "F.Cu") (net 12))
 (segment (start 135.85 97.1) (end 136.25 97.5) (width 0.3) (layer "F.Cu") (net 12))
 (segment (start 172.25 97.5) (end 173.75 97.5) (width 0.3) (layer "F.Cu") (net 8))
 (segment (start 171.85 97.1) (end 172.25 97.5) (width 0.3) (layer "F.Cu") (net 8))
 (segment (start 174.15 97.9) (end 174.15 98.9875) (width 0.3) (layer "F.Cu") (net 8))
 (segment (start 173.75 97.5) (end 174.15 97.9) (width 0.3) (layer "F.Cu") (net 8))
 (segment (start 171.85 96.0125) (end 171.85 97.1) (width 0.3) (layer "F.Cu") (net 8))
 (segment (start 208.25 97.5) (end 209.75 97.5) (width 0.3) (layer "F.Cu") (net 6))
 (segment (start 207.85 96.0125) (end 207.85 97.1) (width 0.3) (layer "F.Cu") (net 6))
 (segment (start 209.75 97.5) (end 210.15 97.9) (width 0.3) (layer "F.Cu") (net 6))
 (segment (start 207.85 97.1) (end 208.25 97.5) (width 0.3) (layer "F.Cu") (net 6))
 (segment (start 210.15 97.9) (end 210.15 98.9875) (width 0.3) (layer "F.Cu") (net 6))
 (segment (start 246.15 97.9) (end 246.15 98.9875) (width 0.3) (layer "F.Cu") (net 1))
 (segment (start 245.75 97.5) (end 246.15 97.9) (width 0.3) (layer "F.Cu") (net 1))
 (segment (start 243.85 96.0125) (end 243.85 97.1) (width 0.3) (layer "F.Cu") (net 1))
 (segment (start 244.25 97.5) (end 245.75 97.5) (width 0.3) (layer "F.Cu") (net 1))
 (segment (start 243.85 97.1) (end 244.25 97.5) (width 0.3) (layer "F.Cu") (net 1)))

